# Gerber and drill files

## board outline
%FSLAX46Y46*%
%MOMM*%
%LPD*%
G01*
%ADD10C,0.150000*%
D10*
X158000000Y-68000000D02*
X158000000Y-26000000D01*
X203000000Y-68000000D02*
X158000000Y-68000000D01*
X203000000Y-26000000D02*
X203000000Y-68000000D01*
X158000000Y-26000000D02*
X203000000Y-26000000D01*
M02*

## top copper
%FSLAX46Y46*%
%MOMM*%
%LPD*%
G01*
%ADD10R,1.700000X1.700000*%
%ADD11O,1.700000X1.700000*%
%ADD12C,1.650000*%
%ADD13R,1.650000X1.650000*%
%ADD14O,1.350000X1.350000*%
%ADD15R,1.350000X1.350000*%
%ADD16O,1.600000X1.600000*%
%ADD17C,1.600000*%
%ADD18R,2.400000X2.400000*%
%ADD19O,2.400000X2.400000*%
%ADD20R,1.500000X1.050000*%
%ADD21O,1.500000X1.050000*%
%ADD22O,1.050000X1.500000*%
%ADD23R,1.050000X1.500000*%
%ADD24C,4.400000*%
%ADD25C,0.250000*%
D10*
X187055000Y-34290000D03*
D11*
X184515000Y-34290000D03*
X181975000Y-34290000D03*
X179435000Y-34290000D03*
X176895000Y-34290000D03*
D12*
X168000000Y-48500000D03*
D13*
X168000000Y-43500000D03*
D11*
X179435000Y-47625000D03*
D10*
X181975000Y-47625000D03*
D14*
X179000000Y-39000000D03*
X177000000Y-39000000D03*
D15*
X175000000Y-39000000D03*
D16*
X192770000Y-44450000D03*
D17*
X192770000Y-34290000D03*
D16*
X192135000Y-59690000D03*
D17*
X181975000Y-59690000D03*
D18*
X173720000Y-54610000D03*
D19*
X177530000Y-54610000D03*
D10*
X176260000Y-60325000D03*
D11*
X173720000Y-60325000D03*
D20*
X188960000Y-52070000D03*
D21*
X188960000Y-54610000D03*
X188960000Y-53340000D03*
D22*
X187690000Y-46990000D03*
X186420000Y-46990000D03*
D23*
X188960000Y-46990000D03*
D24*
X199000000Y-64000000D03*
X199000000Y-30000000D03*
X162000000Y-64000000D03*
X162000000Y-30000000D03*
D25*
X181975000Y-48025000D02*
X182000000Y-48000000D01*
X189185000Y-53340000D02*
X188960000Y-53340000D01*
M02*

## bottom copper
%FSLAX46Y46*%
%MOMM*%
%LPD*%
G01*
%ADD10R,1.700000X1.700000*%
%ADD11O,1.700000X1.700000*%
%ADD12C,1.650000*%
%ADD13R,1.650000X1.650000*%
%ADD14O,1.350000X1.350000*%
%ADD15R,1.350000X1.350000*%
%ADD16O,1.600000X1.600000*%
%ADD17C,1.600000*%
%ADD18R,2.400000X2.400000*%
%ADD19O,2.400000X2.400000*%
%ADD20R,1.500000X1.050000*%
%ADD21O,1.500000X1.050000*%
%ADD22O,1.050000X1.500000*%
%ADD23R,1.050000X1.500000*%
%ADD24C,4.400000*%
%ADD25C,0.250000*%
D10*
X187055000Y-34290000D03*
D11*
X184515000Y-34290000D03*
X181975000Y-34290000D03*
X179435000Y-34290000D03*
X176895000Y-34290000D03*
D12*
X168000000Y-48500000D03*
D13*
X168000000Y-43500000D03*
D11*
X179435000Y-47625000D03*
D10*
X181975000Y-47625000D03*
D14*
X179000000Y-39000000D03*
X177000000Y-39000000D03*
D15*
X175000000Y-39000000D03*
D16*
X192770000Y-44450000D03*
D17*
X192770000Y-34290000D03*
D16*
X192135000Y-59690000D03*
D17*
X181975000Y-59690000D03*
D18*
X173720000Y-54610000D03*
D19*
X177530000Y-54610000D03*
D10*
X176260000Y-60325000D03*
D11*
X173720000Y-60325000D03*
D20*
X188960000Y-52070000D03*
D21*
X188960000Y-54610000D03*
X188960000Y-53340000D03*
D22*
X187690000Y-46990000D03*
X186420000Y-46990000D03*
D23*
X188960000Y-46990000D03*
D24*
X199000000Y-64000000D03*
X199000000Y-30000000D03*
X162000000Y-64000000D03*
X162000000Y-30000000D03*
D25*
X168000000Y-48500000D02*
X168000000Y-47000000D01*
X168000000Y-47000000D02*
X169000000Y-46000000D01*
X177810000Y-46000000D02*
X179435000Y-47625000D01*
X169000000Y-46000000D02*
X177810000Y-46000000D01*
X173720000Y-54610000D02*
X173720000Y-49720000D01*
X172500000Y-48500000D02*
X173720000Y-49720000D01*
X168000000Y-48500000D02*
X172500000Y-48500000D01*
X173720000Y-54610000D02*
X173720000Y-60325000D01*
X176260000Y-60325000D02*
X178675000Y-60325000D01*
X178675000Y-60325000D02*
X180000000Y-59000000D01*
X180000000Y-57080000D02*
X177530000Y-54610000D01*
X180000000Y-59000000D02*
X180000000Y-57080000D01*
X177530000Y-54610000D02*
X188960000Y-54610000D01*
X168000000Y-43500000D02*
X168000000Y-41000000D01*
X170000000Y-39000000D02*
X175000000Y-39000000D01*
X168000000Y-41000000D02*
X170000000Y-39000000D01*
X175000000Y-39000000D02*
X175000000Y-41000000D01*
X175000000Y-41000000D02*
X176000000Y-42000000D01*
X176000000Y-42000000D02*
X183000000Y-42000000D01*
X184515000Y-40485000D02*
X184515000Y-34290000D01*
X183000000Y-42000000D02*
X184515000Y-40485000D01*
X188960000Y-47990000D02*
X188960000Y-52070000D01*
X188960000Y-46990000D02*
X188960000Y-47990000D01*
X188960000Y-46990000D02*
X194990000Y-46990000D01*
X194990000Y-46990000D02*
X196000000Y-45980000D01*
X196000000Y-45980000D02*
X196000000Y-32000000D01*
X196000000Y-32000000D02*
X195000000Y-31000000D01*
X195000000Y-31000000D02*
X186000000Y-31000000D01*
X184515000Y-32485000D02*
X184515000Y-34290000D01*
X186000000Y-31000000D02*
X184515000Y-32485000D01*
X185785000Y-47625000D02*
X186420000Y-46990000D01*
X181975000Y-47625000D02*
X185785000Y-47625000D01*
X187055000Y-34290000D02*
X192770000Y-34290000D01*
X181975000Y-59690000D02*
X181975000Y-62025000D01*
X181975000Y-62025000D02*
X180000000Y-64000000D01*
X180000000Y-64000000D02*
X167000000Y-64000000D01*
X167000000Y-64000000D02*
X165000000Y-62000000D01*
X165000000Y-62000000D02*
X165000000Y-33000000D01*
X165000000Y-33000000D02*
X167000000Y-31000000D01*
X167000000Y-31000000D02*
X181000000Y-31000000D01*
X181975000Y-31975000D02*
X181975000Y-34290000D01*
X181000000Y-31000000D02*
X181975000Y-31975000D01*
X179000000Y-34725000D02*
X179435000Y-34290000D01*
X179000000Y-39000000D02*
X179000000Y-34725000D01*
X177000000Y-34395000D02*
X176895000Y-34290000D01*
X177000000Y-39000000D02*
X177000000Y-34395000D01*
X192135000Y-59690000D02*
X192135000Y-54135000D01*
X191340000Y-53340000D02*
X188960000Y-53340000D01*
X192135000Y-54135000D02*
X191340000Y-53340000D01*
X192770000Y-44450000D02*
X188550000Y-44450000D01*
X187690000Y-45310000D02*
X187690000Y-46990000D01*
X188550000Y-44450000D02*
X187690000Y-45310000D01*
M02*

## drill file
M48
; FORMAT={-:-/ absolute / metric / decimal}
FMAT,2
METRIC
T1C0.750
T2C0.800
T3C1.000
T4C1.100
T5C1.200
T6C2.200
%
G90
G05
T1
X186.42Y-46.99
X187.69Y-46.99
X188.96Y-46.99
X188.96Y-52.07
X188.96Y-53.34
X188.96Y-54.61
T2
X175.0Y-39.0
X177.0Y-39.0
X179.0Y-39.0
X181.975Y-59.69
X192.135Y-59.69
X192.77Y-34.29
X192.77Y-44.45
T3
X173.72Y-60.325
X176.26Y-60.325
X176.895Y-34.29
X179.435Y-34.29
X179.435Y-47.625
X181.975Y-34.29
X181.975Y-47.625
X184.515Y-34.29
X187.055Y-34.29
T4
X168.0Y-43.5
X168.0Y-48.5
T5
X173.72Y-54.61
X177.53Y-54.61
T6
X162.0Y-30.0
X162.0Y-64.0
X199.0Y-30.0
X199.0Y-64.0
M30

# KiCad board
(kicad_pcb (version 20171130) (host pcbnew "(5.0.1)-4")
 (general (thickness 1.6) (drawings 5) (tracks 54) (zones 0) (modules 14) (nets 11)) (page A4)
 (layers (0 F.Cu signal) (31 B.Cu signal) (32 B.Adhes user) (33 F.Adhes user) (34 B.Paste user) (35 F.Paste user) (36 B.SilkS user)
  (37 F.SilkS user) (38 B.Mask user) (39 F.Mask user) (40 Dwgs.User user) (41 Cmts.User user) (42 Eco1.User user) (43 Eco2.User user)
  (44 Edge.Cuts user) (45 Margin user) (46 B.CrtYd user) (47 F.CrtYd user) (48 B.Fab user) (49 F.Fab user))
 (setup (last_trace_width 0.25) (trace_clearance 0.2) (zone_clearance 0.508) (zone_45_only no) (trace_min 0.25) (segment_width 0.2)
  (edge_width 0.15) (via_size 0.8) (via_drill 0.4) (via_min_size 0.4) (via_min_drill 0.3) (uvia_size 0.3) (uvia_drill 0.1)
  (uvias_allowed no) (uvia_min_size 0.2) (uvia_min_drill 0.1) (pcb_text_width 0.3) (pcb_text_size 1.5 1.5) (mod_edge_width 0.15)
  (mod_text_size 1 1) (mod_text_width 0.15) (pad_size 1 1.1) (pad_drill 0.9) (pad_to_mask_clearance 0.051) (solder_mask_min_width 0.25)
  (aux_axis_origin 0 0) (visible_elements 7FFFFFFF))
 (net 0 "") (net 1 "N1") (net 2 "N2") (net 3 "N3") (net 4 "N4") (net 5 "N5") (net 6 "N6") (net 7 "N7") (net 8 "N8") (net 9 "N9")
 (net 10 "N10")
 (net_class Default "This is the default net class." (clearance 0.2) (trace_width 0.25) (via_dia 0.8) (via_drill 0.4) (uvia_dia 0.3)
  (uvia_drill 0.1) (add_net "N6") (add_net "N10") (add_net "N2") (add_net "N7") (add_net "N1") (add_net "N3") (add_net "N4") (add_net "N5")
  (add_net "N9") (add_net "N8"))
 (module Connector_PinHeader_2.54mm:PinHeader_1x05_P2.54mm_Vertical (layer F.Cu) (at 187.055 34.29 270)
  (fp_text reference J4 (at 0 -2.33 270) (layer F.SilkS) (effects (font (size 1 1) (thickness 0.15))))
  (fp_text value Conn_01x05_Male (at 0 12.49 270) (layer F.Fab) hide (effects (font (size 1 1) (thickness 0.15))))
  (pad 1 thru_hole rect (at 0 0 270) (size 1.7 1.7) (drill 1) (layers *.Cu *.Mask) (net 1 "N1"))
  (pad 2 thru_hole oval (at 0 2.54 270) (size 1.7 1.7) (drill 1) (layers *.Cu *.Mask) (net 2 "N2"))
  (pad 3 thru_hole oval (at 0 5.08 270) (size 1.7 1.7) (drill 1) (layers *.Cu *.Mask) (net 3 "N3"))
  (pad 4 thru_hole oval (at 0 7.62 270) (size 1.7 1.7) (drill 1) (layers *.Cu *.Mask) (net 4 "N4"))
  (pad 5 thru_hole oval (at 0 10.16 270) (size 1.7 1.7) (drill 1) (layers *.Cu *.Mask) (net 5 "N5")))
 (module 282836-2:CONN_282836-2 (layer F.Cu) (at 168 46 270)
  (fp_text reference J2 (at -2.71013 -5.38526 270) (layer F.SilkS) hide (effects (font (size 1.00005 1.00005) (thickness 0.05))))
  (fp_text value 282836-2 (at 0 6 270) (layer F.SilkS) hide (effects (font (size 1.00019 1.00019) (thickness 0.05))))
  (pad 2 thru_hole circle (at 2.5 0 270) (size 1.65 1.65) (drill 1.1) (layers *.Cu *.Mask) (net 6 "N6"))
  (pad 1 thru_hole rect (at -2.5 0 270) (size 1.65 1.65) (drill 1.1) (layers *.Cu *.Mask) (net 2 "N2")))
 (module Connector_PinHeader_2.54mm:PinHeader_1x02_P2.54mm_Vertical (layer F.Cu) (at 181.975 47.625 270)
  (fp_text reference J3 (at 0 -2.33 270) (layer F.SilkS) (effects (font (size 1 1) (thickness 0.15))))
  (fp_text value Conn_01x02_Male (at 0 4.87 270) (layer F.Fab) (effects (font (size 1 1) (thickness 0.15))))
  (pad 2 thru_hole oval (at 0 2.54 270) (size 1.7 1.7) (drill 1) (layers *.Cu *.Mask) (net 6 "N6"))
  (pad 1 thru_hole rect (at 0 0 270) (size 1.7 1.7) (drill 1) (layers *.Cu *.Mask) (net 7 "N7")))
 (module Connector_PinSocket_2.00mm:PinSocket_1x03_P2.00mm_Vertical (layer F.Cu) (at 175 39 90)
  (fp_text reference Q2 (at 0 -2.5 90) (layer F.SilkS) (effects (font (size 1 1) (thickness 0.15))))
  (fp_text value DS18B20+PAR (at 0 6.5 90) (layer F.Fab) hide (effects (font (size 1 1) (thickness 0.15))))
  (pad 3 thru_hole oval (at 0 4 90) (size 1.35 1.35) (drill 0.8) (layers *.Cu *.Mask) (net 4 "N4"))
  (pad 2 thru_hole oval (at 0 2 90) (size 1.35 1.35) (drill 0.8) (layers *.Cu *.Mask) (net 5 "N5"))
  (pad 1 thru_hole rect (at 0 0 90) (size 1.35 1.35) (drill 0.8) (layers *.Cu *.Mask) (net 2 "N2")))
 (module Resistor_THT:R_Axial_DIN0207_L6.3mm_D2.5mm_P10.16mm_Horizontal (layer F.Cu) (at 192.77 34.29 270)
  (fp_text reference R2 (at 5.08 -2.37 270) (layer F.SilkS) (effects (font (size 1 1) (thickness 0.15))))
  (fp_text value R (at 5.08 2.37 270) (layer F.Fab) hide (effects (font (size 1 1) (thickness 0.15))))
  (pad 2 thru_hole oval (at 10.16 0 270) (size 1.6 1.6) (drill 0.8) (layers *.Cu *.Mask) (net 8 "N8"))
  (pad 1 thru_hole circle (at 0 0 270) (size 1.6 1.6) (drill 0.8) (layers *.Cu *.Mask) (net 1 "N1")))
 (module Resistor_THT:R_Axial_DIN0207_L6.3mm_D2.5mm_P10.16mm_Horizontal (layer F.Cu) (at 181.975 59.69)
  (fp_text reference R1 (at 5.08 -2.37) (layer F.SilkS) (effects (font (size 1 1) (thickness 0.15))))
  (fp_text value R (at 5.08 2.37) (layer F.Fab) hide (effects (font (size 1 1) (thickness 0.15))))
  (pad 2 thru_hole oval (at 10.16 0) (size 1.6 1.6) (drill 0.8) (layers *.Cu *.Mask) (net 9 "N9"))
  (pad 1 thru_hole circle (at 0 0) (size 1.6 1.6) (drill 0.8) (layers *.Cu *.Mask) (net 3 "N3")))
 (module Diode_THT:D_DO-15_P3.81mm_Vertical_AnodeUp (layer F.Cu) (at 173.72 54.61)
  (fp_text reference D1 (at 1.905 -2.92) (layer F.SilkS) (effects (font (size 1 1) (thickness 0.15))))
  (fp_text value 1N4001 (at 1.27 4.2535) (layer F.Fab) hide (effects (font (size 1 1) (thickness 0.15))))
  (pad 1 thru_hole rect (at 0 0) (size 2.4 2.4) (drill 1.2) (layers *.Cu *.Mask) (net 6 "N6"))
  (pad 2 thru_hole oval (at 3.81 0) (size 2.4 2.4) (drill 1.2) (layers *.Cu *.Mask) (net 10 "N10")))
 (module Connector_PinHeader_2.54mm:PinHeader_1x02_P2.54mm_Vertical (layer F.Cu) (at 176.26 60.325 270)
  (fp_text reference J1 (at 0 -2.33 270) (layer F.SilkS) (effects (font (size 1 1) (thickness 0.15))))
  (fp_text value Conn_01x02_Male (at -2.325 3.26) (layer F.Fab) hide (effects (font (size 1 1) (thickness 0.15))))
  (pad 1 thru_hole rect (at 0 0 270) (size 1.7 1.7) (drill 1) (layers *.Cu *.Mask) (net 10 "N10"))
  (pad 2 thru_hole oval (at 0 2.54 270) (size 1.7 1.7) (drill 1) (layers *.Cu *.Mask) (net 6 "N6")))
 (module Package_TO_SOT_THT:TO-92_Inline (layer F.Cu) (at 188.96 52.07 270)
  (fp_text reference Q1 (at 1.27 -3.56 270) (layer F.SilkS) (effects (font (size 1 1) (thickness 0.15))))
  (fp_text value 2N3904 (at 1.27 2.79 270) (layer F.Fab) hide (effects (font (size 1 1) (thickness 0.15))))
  (pad 1 thru_hole rect (at 0 0 270) (size 1.05 1.5) (drill 0.75) (layers *.Cu *.Mask) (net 2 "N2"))
  (pad 3 thru_hole oval (at 2.54 0 270) (size 1.05 1.5) (drill 0.75) (layers *.Cu *.Mask) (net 10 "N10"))
  (pad 2 thru_hole oval (at 1.27 0 270) (size 1.05 1.5) (drill 0.75) (layers *.Cu *.Mask) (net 9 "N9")))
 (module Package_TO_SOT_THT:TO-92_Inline (layer F.Cu) (at 188.96 46.99 180)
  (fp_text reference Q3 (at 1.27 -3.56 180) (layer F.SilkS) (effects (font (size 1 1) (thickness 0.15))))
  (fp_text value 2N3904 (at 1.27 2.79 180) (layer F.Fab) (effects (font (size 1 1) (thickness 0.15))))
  (pad 2 thru_hole oval (at 1.27 0 180) (size 1.05 1.5) (drill 0.75) (layers *.Cu *.Mask) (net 8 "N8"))
  (pad 3 thru_hole oval (at 2.54 0 180) (size 1.05 1.5) (drill 0.75) (layers *.Cu *.Mask) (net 7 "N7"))
  (pad 1 thru_hole rect (at 0 0 180) (size 1.05 1.5) (drill 0.75) (layers *.Cu *.Mask) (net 2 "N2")))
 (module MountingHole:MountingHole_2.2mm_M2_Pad (layer F.Cu) (at 199 64)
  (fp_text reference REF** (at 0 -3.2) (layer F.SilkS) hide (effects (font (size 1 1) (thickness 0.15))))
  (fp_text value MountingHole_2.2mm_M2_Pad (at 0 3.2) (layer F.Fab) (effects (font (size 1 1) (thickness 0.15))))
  (pad 1 thru_hole circle (at 0 0) (size 4.4 4.4) (drill 2.2) (layers *.Cu *.Mask)))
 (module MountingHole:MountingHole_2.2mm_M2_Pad (layer F.Cu) (at 199 30)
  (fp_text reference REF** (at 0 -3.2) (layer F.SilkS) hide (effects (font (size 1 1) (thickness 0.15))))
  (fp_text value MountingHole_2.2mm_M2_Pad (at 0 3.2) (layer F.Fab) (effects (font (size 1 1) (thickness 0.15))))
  (pad 1 thru_hole circle (at 0 0) (size 4.4 4.4) (drill 2.2) (layers *.Cu *.Mask)))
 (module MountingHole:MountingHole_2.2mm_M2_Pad (layer F.Cu) (at 162 64)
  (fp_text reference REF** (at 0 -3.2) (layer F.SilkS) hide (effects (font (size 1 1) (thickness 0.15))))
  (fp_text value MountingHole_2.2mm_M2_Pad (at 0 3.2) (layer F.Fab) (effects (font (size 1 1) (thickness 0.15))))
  (pad 1 thru_hole circle (at 0 0) (size 4.4 4.4) (drill 2.2) (layers *.Cu *.Mask)))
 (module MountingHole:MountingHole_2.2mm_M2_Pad (layer F.Cu) (at 162 30)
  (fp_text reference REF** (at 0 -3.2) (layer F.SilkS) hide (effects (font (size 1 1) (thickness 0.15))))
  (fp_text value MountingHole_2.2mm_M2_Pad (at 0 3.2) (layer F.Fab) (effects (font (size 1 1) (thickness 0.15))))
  (pad 1 thru_hole circle (at 0 0) (size 4.4 4.4) (drill 2.2) (layers *.Cu *.Mask)))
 (gr_line (start 158 68) (end 158 26) (layer Edge.Cuts) (width 0.15))
 (gr_line (start 203 68) (end 158 68) (layer Edge.Cuts) (width 0.15))
 (gr_line (start 203 26) (end 203 68) (layer Edge.Cuts) (width 0.15))
 (gr_line (start 158 26) (end 203 26) (layer Edge.Cuts) (width 0.15))
 (segment (start 168 48.5) (end 168 47) (width 0.25) (layer B.Cu) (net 6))
 (segment (start 168 47) (end 169 46) (width 0.25) (layer B.Cu) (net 6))
 (segment (start 177.81 46) (end 179.435 47.625) (width 0.25) (layer B.Cu) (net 6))
 (segment (start 169 46) (end 177.81 46) (width 0.25) (layer B.Cu) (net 6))
 (segment (start 173.72 54.61) (end 173.72 49.72) (width 0.25) (layer B.Cu) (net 6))
 (segment (start 172.5 48.5) (end 173.72 49.72) (width 0.25) (layer B.Cu) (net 6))
 (segment (start 168 48.5) (end 172.5 48.5) (width 0.25) (layer B.Cu) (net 6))
 (segment (start 173.72 54.61) (end 173.72 60.325) (width 0.25) (layer B.Cu) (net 6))
 (segment (start 176.26 60.325) (end 178.675 60.325) (width 0.25) (layer B.Cu) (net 10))
 (segment (start 178.675 60.325) (end 180 59) (width 0.25) (layer B.Cu) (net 10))
 (segment (start 180 57.08) (end 177.53 54.61) (width 0.25) (layer B.Cu) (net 10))
 (segment (start 180 59) (end 180 57.08) (width 0.25) (layer B.Cu) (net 10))
 (segment (start 177.53 54.61) (end 188.96 54.61) (width 0.25) (layer B.Cu) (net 10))
 (segment (start 168 43.5) (end 168 41) (width 0.25) (layer B.Cu) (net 2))
 (segment (start 170 39) (end 175 39) (width 0.25) (layer B.Cu) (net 2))
 (segment (start 168 41) (end 170 39) (width 0.25) (layer B.Cu) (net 2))
 (segment (start 175 39) (end 175 41) (width 0.25) (layer B.Cu) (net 2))
 (segment (start 175 41) (end 176 42) (width 0.25) (layer B.Cu) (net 2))
 (segment (start 176 42) (end 183 42) (width 0.25) (layer B.Cu) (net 2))
 (segment (start 184.515 40.485) (end 184.515 34.29) (width 0.25) (layer B.Cu) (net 2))
 (segment (start 183 42) (end 184.515 40.485) (width 0.25) (layer B.Cu) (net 2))
 (segment (start 188.96 47.99) (end 188.96 52.07) (width 0.25) (layer B.Cu) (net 2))
 (segment (start 188.96 46.99) (end 188.96 47.99) (width 0.25) (layer B.Cu) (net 2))
 (segment (start 188.96 46.99) (end 194.99 46.99) (width 0.25) (layer B.Cu) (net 2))
 (segment (start 194.99 46.99) (end 196 45.98) (width 0.25) (layer B.Cu) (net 2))
 (segment (start 196 45.98) (end 196 32) (width 0.25) (layer B.Cu) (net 2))
 (segment (start 196 32) (end 195 31) (width 0.25) (layer B.Cu) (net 2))
 (segment (start 195 31) (end 186 31) (width 0.25) (layer B.Cu) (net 2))
 (segment (start 184.515 32.485) (end 184.515 34.29) (width 0.25) (layer B.Cu) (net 2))
 (segment (start 186 31) (end 184.515 32.485) (width 0.25) (layer B.Cu) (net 2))
 (segment (start 181.975 48.025) (end 182 48) (width 0.25) (layer F.Cu) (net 7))
 (segment (start 185.785 47.625) (end 186.42 46.99) (width 0.25) (layer B.Cu) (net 7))
 (segment (start 181.975 47.625) (end 185.785 47.625) (width 0.25) (layer B.Cu) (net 7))
 (segment (start 187.055 34.29) (end 192.77 34.29) (width 0.25) (layer B.Cu) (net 1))
 (segment (start 181.975 59.69) (end 181.975 62.025) (width 0.25) (layer B.Cu) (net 3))
 (segment (start 181.975 62.025) (end 180 64) (width 0.25) (layer B.Cu) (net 3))
 (segment (start 180 64) (end 167 64) (width 0.25) (layer B.Cu) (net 3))
 (segment (start 167 64) (end 165 62) (width 0.25) (layer B.Cu) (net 3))
 (segment (start 165 62) (end 165 33) (width 0.25) (layer B.Cu) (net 3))
 (segment (start 165 33) (end 167 31) (width 0.25) (layer B.Cu) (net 3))
 (segment (start 167 31) (end 181 31) (width 0.25) (layer B.Cu) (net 3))
 (segment (start 181.975 31.975) (end 181.975 34.29) (width 0.25) (layer B.Cu) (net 3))
 (segment (start 181 31) (end 181.975 31.975) (width 0.25) (layer B.Cu) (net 3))
 (segment (start 179 34.725) (end 179.435 34.29) (width 0.25) (layer B.Cu) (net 4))
 (segment (start 179 39) (end 179 34.725) (width 0.25) (layer B.Cu) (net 4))
 (segment (start 177 34.395) (end 176.895 34.29) (width 0.25) (layer B.Cu) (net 5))
 (segment (start 177 39) (end 177 34.395) (width 0.25) (layer B.Cu) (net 5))
 (segment (start 189.185 53.34) (end 188.96 53.34) (width 0.25) (layer F.Cu) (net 9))
 (segment (start 192.135 59.69) (end 192.135 54.135) (width 0.25) (layer B.Cu) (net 9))
 (segment (start 191.34 53.34) (end 188.96 53.34) (width 0.25) (layer B.Cu) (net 9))
 (segment (start 192.135 54.135) (end 191.34 53.34) (width 0.25) (layer B.Cu) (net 9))
 (segment (start 192.77 44.45) (end 188.55 44.45) (width 0.25) (layer B.Cu) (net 8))
 (segment (start 187.69 45.31) (end 187.69 46.99) (width 0.25) (layer B.Cu) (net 8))
 (segment (start 188.55 44.45) (end 187.69 45.31) (width 0.25) (layer B.Cu) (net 8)))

